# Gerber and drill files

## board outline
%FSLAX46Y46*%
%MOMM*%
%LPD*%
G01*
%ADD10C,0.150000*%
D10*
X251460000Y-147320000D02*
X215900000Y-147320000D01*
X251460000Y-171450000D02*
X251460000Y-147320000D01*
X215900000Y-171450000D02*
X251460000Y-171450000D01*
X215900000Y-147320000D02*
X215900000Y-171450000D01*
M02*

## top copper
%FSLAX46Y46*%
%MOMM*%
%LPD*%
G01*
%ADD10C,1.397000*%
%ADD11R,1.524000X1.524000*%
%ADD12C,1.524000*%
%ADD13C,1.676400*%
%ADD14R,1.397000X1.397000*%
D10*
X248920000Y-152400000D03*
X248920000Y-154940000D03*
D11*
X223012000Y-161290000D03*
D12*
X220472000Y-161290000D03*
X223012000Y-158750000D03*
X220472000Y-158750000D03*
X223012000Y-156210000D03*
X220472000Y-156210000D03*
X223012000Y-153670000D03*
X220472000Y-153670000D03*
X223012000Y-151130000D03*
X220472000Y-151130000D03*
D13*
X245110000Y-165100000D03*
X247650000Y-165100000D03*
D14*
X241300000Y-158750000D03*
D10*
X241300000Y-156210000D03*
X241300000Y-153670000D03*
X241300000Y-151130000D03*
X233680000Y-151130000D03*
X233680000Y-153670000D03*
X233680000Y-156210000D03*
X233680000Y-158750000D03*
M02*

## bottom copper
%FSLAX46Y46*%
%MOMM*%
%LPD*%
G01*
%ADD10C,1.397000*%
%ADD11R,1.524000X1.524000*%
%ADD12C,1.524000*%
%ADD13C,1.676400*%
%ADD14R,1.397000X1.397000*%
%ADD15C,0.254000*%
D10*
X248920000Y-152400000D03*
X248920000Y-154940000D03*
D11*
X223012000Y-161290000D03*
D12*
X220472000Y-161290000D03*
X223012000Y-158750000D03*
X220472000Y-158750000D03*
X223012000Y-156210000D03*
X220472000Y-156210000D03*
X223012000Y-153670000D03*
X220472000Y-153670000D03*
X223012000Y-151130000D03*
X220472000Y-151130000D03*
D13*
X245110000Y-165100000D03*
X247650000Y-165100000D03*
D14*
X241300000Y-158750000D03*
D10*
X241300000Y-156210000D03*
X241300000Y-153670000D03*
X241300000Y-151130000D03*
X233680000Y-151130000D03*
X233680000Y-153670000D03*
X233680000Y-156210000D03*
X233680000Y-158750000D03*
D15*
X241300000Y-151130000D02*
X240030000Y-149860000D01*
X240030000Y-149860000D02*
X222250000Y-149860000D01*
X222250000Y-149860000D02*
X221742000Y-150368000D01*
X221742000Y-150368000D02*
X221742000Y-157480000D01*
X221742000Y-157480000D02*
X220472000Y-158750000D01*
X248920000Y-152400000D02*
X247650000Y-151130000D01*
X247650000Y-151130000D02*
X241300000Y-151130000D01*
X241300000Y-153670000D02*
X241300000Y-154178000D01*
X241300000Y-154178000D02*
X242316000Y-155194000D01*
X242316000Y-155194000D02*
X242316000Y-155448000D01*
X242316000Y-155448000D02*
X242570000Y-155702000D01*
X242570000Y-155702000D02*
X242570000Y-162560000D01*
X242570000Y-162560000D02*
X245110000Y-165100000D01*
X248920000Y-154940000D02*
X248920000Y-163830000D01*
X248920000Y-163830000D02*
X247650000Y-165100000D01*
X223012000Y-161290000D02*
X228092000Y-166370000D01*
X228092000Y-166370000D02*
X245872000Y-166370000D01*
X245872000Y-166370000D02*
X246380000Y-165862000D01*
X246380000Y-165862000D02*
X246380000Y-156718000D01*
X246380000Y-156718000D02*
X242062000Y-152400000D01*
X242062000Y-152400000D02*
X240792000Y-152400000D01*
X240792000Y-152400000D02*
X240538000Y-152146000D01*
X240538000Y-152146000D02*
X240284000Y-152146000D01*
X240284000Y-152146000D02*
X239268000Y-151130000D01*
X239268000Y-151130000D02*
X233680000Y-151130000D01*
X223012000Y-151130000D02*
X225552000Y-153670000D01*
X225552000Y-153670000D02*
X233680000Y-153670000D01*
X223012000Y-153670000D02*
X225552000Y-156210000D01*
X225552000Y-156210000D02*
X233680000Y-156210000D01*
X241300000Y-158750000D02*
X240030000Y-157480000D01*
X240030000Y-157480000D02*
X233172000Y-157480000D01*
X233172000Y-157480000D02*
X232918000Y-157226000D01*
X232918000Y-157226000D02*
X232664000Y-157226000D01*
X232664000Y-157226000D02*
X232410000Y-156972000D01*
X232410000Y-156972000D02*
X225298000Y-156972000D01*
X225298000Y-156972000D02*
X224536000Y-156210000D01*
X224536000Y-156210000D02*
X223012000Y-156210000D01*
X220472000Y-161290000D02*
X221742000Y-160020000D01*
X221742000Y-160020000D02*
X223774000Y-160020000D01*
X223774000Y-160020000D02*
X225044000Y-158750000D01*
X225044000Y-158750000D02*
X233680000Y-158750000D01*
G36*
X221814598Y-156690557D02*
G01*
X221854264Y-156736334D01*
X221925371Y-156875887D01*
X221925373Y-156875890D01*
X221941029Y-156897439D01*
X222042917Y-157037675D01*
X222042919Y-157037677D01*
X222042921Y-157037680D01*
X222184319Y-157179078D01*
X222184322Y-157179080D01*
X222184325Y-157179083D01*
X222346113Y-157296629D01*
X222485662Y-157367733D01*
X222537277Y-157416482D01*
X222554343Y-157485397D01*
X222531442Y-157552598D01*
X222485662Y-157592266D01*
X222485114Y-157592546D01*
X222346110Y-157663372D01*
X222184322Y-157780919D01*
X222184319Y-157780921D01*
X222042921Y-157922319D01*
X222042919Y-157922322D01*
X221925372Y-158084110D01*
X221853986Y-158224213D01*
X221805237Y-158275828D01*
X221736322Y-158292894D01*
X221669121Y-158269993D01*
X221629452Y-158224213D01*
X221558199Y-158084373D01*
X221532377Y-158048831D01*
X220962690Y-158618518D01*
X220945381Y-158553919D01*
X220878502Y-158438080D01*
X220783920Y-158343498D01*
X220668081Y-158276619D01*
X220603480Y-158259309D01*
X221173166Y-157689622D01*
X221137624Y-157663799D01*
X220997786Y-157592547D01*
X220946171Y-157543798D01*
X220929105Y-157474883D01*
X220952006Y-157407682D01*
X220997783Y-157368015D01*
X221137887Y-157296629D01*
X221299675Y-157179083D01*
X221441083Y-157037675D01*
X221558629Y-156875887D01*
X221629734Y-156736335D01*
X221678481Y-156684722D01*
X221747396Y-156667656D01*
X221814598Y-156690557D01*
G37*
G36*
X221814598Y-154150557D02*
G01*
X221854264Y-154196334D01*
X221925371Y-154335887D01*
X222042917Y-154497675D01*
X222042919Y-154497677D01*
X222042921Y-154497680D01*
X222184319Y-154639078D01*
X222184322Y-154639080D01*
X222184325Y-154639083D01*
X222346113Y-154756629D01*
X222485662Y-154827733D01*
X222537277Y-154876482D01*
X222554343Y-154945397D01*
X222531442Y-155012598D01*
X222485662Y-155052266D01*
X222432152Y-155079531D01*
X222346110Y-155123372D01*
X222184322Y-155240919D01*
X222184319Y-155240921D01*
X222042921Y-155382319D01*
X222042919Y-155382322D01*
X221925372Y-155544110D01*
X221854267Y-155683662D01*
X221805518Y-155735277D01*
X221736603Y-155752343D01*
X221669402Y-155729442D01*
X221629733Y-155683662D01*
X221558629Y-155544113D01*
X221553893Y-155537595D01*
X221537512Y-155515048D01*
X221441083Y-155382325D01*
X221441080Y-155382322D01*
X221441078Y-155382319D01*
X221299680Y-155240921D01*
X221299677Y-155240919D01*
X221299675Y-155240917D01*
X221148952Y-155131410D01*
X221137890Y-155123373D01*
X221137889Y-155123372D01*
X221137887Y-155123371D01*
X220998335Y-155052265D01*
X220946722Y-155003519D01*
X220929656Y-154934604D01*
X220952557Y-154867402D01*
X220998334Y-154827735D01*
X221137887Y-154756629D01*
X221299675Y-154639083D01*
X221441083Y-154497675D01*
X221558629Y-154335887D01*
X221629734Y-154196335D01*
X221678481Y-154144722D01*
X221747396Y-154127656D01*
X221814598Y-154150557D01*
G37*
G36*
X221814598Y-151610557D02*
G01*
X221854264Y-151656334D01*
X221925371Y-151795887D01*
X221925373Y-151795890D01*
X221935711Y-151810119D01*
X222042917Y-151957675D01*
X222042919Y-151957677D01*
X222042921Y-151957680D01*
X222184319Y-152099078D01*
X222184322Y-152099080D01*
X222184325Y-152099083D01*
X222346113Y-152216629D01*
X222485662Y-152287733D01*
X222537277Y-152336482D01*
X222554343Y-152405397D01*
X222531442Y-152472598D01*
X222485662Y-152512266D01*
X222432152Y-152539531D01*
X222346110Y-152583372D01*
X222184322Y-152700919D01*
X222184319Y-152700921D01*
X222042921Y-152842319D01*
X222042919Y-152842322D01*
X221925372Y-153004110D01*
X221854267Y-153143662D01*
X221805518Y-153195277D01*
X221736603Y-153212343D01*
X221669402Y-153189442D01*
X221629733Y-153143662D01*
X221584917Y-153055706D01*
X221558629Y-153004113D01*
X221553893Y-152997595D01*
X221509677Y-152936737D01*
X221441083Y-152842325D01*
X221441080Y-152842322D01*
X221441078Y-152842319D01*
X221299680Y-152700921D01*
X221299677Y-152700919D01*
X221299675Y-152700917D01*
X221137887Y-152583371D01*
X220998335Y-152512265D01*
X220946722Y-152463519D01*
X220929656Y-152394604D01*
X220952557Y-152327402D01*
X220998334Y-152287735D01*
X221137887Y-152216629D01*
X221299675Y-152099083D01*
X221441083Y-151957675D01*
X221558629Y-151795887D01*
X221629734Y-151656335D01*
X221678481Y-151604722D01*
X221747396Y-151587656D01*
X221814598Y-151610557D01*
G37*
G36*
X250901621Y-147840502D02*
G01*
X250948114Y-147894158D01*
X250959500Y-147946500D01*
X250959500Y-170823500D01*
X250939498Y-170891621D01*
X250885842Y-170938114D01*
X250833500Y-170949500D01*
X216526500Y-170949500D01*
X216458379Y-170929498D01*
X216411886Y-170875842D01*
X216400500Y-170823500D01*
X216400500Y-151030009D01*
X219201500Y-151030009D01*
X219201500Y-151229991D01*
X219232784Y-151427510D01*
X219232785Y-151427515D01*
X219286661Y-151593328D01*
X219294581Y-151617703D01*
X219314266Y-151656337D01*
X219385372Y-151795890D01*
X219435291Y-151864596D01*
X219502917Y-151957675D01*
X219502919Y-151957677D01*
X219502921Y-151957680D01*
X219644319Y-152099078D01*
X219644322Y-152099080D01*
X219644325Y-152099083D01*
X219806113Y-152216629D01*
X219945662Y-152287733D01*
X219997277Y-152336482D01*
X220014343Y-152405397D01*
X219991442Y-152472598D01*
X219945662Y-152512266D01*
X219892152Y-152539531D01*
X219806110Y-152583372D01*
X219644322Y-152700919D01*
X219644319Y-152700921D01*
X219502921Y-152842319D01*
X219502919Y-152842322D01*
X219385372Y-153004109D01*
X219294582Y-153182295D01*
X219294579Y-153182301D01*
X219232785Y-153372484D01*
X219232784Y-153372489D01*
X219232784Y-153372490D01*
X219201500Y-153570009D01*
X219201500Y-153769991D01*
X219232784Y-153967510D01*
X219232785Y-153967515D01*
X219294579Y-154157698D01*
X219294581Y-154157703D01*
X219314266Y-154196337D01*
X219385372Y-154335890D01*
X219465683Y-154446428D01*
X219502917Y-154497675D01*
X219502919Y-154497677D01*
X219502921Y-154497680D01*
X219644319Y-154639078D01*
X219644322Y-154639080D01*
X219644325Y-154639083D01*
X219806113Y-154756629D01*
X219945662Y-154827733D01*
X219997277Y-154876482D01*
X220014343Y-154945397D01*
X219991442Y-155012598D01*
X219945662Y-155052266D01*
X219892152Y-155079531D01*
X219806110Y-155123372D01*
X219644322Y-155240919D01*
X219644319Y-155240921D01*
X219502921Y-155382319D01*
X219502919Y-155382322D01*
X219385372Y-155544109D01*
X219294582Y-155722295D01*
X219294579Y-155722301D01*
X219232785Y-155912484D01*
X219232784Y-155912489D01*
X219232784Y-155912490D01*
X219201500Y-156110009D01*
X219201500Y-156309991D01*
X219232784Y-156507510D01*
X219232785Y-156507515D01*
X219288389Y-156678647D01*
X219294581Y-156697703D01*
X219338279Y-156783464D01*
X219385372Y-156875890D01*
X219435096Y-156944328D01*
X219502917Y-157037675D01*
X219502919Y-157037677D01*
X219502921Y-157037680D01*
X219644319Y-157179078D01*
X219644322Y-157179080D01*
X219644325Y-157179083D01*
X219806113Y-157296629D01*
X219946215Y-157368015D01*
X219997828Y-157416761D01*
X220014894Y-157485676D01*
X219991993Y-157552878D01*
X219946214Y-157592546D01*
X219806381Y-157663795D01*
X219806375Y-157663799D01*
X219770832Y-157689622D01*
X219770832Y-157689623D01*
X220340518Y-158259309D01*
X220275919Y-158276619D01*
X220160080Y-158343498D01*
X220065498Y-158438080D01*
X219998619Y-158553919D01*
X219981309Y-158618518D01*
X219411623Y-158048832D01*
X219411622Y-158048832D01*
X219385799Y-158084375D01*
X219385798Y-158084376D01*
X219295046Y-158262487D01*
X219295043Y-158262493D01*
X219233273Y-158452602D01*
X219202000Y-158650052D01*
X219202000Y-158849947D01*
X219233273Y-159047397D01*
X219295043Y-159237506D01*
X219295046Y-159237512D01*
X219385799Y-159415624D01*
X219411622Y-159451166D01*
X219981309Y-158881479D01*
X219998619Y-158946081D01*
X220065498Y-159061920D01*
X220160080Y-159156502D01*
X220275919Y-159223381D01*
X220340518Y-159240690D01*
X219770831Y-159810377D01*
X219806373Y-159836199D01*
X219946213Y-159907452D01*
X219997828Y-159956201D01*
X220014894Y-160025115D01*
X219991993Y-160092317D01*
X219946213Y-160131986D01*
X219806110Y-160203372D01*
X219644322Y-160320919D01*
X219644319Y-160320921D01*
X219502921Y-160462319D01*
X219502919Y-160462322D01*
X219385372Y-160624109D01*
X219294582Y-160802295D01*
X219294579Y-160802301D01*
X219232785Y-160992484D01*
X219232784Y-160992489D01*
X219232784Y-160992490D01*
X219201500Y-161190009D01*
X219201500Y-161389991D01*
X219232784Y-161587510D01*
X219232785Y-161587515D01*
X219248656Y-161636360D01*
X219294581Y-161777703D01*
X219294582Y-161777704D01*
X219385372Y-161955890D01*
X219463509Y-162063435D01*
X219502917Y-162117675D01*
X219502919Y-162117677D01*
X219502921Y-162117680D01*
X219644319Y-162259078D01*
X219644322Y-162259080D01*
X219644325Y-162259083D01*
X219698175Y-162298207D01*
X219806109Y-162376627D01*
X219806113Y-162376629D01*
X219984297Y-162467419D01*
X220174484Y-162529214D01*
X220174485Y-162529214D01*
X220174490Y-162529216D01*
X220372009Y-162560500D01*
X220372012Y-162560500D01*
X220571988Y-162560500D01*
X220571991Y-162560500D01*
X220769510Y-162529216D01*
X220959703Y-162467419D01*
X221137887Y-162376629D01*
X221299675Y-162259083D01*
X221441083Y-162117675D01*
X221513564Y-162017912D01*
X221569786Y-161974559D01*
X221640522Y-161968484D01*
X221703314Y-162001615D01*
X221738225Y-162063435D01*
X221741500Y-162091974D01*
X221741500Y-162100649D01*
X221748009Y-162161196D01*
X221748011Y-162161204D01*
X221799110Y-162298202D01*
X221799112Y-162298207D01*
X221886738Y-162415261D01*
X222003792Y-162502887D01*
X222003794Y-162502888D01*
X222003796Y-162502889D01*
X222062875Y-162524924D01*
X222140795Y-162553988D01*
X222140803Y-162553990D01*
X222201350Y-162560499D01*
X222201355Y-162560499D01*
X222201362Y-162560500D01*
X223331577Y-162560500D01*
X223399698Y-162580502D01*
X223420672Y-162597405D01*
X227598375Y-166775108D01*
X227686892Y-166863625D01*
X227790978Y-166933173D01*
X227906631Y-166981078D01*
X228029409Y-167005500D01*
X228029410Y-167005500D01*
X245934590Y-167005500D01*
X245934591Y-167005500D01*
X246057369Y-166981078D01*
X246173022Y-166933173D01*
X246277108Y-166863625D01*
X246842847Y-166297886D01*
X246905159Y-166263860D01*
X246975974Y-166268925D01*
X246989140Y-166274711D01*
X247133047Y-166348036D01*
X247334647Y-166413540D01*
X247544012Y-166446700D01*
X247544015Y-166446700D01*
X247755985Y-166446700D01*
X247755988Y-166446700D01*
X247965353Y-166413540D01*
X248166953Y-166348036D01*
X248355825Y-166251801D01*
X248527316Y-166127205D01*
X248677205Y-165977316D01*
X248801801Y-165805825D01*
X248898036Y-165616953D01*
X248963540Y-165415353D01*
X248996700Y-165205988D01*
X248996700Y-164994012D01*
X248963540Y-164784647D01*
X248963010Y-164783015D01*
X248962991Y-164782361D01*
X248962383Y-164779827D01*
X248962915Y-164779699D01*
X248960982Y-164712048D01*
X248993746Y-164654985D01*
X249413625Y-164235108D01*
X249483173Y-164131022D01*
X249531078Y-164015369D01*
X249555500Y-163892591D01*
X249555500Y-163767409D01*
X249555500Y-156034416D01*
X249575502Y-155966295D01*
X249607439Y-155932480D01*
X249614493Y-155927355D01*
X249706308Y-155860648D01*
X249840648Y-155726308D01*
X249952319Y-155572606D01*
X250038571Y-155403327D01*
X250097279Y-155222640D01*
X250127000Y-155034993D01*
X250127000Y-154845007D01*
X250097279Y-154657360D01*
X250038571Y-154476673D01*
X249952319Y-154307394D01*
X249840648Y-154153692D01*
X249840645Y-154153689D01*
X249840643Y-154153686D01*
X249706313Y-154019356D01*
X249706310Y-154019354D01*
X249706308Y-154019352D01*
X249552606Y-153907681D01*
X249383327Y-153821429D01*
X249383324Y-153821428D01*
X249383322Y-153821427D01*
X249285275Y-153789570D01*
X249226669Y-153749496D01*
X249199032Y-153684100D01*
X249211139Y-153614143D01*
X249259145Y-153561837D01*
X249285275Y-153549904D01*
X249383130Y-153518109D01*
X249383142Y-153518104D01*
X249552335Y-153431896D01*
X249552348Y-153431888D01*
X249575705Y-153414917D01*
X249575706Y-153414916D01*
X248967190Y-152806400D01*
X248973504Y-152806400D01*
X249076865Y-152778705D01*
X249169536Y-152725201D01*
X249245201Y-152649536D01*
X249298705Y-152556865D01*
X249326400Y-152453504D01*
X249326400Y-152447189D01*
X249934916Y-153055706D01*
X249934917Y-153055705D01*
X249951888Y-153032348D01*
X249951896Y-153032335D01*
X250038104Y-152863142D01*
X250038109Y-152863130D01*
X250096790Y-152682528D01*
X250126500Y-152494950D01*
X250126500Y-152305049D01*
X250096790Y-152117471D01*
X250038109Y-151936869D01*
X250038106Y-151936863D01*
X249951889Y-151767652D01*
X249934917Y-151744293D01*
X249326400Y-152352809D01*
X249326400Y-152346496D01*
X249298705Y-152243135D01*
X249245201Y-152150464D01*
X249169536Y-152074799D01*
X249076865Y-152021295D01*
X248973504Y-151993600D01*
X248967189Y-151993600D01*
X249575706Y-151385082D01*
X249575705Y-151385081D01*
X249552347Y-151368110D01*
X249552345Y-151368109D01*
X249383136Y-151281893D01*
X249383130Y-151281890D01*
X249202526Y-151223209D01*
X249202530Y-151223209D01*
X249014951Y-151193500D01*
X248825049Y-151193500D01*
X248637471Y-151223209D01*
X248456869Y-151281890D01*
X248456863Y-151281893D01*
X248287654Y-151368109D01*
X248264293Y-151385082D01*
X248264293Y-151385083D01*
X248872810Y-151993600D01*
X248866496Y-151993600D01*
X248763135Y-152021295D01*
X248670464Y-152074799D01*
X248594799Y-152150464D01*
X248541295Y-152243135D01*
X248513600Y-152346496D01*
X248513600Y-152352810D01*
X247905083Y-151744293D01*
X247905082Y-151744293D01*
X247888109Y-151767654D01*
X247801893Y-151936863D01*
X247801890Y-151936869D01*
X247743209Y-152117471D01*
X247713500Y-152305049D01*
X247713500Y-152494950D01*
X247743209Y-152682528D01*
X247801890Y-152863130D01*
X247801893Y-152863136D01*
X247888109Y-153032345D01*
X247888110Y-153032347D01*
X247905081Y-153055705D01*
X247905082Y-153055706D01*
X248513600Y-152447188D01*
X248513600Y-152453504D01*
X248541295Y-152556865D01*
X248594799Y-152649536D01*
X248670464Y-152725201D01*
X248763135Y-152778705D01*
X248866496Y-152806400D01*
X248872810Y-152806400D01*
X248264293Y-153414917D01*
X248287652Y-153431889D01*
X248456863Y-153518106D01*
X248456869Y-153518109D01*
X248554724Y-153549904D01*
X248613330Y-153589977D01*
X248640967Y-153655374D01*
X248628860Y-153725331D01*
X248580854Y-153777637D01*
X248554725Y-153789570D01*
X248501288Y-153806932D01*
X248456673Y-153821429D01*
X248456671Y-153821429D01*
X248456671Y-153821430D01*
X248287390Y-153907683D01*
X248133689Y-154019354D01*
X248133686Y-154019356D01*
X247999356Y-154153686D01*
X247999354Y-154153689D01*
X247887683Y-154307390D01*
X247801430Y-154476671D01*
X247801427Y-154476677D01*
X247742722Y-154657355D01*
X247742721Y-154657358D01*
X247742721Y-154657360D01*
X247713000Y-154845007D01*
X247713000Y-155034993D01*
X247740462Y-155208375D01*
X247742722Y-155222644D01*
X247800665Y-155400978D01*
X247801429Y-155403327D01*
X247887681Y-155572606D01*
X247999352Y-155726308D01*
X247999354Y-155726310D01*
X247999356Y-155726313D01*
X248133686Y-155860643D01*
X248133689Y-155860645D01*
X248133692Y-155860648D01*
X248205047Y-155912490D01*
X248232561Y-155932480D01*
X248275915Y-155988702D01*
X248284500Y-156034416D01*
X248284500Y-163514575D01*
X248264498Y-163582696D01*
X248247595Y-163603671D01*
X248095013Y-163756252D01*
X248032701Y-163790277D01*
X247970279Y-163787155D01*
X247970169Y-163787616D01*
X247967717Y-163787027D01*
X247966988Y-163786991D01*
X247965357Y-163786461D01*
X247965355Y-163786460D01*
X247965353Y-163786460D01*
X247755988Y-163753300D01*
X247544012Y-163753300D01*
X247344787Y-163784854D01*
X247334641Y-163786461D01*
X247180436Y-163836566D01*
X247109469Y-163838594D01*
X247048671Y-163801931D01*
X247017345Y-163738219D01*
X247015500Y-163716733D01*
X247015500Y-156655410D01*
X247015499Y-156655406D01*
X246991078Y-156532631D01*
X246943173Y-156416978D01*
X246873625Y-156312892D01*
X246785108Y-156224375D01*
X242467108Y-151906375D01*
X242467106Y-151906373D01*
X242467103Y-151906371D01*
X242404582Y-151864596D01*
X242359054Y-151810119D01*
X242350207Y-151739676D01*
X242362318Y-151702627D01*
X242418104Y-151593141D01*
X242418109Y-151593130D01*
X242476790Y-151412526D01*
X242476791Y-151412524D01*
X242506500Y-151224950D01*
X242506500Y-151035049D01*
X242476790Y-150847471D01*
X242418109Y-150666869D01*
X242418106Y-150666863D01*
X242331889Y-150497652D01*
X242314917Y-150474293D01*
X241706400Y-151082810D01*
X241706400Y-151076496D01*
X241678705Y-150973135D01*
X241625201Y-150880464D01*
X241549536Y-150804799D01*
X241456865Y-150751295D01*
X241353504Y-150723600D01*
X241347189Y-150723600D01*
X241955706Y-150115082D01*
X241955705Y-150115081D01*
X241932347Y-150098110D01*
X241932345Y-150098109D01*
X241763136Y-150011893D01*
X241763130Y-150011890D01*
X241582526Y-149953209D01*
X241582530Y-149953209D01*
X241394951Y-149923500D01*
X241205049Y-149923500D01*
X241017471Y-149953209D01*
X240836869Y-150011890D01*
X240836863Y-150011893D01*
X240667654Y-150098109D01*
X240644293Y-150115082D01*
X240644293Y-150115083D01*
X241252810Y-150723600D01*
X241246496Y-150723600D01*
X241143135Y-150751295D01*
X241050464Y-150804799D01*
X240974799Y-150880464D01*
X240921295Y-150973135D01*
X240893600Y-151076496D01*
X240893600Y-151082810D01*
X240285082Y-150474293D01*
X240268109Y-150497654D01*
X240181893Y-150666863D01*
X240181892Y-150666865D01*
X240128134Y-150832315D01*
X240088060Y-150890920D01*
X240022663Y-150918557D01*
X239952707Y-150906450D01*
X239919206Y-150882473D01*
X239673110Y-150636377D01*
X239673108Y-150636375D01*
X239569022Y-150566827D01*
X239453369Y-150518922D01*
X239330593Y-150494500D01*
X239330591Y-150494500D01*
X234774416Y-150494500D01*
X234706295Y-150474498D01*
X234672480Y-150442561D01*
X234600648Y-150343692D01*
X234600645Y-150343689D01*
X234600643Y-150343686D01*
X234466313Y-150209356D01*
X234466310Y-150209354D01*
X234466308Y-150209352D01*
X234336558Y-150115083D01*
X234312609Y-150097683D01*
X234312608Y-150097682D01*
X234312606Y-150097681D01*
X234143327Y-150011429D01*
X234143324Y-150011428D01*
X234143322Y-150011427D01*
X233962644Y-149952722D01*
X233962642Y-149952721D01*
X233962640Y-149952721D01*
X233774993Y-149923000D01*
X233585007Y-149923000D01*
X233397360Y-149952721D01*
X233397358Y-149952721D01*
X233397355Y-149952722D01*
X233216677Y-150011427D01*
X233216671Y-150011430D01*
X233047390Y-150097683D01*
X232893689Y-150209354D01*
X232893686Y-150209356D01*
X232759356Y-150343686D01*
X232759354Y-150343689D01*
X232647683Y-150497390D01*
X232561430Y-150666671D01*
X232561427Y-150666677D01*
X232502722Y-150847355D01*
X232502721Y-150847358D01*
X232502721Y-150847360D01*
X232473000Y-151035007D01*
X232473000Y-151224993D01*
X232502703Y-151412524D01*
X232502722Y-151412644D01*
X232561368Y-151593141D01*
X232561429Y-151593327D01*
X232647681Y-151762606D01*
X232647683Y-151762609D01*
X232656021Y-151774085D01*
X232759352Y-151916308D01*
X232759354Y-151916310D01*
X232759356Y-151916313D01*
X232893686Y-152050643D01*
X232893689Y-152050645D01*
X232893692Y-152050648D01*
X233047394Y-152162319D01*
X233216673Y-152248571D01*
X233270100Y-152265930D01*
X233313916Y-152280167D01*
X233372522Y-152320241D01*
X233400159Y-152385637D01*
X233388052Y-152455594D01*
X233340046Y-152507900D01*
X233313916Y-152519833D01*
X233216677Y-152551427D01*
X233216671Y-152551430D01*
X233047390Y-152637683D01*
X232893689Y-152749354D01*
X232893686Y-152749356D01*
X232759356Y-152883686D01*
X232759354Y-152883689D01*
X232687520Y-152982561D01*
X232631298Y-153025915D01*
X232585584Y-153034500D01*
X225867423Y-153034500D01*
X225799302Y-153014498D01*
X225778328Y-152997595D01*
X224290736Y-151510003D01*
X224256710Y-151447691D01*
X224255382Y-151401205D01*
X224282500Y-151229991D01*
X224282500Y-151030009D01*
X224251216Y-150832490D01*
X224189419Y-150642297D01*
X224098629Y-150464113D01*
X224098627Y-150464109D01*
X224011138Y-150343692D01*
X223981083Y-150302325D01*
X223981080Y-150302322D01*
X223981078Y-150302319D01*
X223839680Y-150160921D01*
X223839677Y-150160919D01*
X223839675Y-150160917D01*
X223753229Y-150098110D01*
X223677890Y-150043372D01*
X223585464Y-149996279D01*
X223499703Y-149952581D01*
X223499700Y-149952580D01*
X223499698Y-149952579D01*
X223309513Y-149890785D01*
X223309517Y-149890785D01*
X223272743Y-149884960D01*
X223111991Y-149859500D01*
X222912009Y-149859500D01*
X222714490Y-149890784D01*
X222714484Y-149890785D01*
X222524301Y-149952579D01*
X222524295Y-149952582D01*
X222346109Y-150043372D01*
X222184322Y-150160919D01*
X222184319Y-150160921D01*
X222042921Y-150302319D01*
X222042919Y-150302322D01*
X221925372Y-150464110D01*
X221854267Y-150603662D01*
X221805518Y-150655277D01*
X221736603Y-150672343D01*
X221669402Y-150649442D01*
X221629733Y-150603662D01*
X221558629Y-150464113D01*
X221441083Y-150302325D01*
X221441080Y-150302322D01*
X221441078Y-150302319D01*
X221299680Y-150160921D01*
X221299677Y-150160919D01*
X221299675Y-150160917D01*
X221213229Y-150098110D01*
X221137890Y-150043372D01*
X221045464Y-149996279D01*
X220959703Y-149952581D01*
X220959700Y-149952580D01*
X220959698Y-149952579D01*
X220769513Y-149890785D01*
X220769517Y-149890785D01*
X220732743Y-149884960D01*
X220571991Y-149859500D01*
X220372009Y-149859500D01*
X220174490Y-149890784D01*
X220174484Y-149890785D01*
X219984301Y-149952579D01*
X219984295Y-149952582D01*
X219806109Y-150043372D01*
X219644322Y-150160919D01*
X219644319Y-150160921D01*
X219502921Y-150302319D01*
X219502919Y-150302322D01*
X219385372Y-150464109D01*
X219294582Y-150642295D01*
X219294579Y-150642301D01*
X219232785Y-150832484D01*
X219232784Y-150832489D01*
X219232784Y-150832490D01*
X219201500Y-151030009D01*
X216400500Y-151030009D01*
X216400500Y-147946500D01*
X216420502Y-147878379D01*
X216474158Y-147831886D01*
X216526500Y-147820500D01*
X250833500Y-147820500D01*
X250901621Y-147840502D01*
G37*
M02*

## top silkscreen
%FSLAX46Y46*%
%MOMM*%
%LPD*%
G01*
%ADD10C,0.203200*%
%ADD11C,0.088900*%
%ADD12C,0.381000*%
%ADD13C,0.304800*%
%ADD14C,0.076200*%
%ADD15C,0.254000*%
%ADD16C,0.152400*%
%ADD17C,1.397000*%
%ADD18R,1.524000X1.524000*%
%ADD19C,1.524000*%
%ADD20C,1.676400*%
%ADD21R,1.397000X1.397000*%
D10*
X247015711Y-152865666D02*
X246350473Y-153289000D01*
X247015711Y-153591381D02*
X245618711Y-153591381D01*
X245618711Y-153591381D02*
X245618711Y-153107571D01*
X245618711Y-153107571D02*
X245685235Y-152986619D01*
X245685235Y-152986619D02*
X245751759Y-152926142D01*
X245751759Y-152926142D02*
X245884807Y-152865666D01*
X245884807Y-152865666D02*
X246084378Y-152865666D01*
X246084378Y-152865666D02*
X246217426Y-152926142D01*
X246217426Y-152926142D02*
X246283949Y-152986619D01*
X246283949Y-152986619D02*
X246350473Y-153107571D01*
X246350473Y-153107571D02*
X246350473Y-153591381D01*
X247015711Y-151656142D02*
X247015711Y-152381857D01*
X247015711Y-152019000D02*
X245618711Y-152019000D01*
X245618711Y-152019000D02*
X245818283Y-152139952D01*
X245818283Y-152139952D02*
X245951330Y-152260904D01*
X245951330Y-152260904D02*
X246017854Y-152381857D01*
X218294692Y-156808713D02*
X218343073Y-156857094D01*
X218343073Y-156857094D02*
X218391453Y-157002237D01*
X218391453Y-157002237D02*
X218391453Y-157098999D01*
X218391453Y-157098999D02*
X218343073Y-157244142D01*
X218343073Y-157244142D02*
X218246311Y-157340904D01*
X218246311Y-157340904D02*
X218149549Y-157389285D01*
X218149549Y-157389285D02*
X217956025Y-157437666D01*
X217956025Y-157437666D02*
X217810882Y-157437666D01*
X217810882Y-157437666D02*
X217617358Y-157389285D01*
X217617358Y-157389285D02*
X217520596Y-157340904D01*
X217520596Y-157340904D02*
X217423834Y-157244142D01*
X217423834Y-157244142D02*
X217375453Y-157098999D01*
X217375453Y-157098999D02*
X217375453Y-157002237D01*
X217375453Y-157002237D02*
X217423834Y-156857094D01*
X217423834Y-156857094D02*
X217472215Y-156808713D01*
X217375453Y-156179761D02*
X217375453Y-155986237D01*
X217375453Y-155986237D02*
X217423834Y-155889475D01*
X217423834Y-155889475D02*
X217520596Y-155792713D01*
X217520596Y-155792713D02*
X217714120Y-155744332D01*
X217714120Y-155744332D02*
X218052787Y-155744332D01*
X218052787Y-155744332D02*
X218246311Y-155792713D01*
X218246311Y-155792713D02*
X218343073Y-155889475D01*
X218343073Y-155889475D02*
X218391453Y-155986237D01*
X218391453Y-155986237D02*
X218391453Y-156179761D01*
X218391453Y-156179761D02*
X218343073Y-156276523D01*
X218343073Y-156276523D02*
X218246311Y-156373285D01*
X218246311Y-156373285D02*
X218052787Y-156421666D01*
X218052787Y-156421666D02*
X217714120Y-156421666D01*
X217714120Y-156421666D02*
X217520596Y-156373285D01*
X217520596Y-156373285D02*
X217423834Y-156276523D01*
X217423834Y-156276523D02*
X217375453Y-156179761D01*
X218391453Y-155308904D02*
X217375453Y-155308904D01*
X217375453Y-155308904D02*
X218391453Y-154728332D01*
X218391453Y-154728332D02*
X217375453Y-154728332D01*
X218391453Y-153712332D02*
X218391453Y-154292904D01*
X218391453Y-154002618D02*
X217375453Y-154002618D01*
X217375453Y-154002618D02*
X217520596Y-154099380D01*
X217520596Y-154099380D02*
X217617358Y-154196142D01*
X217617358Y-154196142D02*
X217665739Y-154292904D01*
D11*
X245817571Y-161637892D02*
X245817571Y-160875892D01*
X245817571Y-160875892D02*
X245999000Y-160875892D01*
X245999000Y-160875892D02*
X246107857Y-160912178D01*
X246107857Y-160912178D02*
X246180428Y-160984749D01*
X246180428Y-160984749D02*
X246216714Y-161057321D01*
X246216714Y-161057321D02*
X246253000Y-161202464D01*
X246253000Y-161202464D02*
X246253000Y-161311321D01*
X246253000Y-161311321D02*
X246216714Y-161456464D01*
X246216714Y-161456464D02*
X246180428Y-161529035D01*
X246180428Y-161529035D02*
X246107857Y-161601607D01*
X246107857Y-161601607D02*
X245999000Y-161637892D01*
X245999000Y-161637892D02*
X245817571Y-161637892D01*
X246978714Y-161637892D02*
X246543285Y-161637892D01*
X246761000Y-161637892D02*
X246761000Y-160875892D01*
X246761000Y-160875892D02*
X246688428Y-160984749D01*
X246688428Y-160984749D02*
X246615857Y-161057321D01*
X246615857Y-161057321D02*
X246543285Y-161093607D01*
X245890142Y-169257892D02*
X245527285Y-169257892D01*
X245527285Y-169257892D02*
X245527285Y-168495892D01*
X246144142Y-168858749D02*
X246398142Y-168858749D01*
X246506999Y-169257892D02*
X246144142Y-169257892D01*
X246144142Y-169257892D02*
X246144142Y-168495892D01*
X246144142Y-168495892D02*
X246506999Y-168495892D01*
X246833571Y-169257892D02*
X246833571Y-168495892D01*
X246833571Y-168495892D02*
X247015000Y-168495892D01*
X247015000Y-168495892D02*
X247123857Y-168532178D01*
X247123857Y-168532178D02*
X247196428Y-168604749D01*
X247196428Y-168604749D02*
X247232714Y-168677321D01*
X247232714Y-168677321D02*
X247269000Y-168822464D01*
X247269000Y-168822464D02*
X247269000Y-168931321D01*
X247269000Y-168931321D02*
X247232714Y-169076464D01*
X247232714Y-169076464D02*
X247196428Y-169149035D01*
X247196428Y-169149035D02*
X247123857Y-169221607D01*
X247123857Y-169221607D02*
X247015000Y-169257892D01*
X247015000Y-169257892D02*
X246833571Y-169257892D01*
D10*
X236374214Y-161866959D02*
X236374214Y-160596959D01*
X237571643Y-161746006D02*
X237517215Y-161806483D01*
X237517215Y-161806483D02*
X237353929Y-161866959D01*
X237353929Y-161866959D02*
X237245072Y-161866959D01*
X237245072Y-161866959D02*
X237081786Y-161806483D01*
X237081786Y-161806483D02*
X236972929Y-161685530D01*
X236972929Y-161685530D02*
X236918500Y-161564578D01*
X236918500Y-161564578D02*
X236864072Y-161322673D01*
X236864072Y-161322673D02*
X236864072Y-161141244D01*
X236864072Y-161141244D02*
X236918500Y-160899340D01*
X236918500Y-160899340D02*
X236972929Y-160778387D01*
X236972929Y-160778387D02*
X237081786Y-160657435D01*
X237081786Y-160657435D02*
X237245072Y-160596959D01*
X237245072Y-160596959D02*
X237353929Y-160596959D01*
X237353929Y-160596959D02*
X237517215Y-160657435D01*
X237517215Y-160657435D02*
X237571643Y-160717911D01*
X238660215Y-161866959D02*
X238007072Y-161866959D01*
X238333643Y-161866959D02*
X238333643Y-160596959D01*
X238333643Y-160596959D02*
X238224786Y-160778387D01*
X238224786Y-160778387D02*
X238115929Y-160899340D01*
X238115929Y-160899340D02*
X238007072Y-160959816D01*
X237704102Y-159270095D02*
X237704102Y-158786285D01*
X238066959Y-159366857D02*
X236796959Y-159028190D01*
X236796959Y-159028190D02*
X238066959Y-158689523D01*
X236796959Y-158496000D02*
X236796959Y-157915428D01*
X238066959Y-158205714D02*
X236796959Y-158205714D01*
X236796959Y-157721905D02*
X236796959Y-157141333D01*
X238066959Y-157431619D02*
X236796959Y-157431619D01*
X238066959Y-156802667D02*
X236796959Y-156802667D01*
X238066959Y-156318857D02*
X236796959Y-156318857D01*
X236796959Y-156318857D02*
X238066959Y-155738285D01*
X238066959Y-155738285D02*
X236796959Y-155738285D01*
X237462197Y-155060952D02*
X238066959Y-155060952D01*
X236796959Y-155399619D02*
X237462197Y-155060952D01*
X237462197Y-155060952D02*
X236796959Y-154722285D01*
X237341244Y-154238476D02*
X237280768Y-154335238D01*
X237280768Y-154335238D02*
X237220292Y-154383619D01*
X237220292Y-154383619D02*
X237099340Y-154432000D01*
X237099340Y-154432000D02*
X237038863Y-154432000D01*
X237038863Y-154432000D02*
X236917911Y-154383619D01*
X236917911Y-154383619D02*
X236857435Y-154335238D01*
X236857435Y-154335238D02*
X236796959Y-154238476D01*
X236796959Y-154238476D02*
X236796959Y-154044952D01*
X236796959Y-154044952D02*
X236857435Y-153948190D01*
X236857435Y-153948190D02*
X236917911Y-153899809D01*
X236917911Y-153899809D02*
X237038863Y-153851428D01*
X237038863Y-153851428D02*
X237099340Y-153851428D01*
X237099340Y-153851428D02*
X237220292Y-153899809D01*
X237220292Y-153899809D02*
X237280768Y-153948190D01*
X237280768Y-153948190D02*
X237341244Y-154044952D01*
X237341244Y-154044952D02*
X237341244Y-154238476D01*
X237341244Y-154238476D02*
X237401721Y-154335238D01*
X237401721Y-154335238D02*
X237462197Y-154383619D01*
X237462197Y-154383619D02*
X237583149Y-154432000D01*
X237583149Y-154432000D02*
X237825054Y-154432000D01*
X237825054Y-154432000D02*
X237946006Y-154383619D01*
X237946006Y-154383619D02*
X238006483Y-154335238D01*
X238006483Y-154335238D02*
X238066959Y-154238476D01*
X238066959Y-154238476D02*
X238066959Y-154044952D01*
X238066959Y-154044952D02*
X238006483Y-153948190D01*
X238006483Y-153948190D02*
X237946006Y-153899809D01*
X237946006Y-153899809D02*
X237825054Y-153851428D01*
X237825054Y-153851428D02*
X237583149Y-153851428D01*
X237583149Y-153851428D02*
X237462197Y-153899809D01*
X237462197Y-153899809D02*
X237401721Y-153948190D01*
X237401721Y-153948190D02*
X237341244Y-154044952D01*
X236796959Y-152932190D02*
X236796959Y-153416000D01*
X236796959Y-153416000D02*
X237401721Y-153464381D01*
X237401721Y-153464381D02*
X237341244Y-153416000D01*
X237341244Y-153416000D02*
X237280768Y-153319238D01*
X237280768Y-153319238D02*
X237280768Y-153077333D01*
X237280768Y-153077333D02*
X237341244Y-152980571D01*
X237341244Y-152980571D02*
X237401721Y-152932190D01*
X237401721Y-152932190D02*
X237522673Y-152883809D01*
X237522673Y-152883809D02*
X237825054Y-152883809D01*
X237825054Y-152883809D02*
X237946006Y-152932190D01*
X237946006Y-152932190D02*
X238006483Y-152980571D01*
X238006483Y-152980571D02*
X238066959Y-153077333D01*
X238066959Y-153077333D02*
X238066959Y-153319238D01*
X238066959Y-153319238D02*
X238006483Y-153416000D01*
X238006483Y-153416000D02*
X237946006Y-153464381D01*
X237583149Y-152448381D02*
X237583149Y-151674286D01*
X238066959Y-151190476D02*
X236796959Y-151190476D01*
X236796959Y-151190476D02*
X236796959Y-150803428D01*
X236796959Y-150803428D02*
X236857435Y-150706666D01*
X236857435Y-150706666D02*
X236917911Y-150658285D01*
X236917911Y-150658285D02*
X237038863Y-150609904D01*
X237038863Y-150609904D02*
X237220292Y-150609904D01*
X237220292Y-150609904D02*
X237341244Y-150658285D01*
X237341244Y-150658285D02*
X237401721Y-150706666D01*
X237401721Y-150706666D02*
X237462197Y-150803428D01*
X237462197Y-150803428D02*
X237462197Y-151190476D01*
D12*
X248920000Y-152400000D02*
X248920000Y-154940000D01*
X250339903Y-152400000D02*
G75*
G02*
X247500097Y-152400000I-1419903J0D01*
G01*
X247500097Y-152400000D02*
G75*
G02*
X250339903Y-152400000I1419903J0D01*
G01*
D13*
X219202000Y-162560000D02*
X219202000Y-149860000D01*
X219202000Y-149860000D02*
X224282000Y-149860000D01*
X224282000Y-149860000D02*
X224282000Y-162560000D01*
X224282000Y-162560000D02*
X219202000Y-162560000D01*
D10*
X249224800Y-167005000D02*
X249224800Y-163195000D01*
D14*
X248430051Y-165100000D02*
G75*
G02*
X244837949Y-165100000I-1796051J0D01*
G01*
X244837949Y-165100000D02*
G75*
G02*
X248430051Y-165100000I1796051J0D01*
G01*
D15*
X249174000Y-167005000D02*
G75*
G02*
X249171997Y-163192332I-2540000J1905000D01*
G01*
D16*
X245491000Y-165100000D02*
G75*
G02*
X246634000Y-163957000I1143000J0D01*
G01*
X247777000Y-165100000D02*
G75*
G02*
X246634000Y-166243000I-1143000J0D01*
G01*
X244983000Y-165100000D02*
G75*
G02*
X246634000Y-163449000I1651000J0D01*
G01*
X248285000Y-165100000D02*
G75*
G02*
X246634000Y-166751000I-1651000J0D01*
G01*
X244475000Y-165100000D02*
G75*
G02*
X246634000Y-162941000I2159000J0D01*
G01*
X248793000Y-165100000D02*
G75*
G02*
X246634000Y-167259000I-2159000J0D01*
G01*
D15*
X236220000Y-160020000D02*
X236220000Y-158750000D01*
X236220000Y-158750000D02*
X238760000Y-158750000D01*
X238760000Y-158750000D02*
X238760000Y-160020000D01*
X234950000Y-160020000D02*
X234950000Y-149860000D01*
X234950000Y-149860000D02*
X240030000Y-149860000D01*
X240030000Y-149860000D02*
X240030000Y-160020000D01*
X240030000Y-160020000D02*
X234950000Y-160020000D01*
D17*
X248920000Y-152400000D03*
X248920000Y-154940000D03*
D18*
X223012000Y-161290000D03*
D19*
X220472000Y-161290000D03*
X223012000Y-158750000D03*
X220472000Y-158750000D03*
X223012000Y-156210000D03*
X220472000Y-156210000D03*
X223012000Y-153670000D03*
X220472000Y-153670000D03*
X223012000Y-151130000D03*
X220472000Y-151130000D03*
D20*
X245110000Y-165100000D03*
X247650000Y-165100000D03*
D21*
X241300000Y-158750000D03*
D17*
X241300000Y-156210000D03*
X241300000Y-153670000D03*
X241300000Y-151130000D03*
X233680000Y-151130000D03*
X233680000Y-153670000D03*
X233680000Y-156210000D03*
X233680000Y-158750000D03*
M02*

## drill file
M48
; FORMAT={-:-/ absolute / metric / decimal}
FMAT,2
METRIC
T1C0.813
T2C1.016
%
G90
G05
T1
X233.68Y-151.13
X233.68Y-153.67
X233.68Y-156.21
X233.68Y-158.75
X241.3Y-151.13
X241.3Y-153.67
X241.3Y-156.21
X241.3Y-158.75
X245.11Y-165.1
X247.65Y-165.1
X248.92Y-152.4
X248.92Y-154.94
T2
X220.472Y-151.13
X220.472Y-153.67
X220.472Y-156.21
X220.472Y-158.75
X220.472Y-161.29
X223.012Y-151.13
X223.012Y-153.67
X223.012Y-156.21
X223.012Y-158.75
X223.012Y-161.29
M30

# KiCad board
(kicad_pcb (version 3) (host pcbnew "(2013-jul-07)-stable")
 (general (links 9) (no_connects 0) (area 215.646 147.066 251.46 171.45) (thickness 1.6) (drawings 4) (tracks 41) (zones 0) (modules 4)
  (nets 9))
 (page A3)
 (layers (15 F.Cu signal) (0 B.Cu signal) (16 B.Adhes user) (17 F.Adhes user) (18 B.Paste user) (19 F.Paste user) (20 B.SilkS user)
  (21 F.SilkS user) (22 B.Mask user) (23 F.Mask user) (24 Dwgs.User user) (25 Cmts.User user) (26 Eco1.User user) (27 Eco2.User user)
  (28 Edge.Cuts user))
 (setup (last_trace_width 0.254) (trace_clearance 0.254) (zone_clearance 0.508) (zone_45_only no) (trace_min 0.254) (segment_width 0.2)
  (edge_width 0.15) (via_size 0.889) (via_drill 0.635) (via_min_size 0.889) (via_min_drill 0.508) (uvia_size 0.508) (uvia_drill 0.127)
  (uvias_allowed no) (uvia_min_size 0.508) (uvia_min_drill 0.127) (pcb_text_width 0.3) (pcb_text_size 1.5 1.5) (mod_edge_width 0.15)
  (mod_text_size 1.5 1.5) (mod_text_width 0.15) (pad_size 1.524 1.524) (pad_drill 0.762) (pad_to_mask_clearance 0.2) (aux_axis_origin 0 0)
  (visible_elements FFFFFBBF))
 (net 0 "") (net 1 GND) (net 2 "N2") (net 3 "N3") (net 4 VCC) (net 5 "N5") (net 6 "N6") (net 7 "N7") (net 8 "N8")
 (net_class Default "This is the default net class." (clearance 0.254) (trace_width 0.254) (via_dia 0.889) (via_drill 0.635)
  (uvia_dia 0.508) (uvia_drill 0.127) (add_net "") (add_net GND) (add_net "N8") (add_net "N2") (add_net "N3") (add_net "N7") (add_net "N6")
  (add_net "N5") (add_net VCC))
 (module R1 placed (layer F.Cu) (at 248.92 153.67 270) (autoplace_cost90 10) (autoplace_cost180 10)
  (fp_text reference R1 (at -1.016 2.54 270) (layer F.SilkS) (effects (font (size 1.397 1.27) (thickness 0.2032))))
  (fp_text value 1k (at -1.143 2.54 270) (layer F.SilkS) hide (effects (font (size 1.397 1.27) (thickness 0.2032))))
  (fp_line (start -1.27 0) (end 1.27 0) (layer F.SilkS) (width 0.381))
  (fp_circle (center -1.27 0) (end -0.635 1.27) (layer F.SilkS) (width 0.381))
  (pad 1 thru_hole circle (at -1.27 0 270) (size 1.397 1.397) (drill 0.8128) (layers *.Cu *.Mask F.SilkS) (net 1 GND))
  (pad 2 thru_hole circle (at 1.27 0 270) (size 1.397 1.397) (drill 0.8128) (layers *.Cu *.Mask F.SilkS) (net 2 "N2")))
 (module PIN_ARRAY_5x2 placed (layer F.Cu) (at 221.742 156.21 90)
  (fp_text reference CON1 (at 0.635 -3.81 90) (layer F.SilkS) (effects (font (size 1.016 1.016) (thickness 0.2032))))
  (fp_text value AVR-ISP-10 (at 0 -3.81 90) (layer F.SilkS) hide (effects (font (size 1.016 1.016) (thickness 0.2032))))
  (fp_line (start -6.35 -2.54) (end 6.35 -2.54) (layer F.SilkS) (width 0.3048))
  (fp_line (start 6.35 -2.54) (end 6.35 2.54) (layer F.SilkS) (width 0.3048))
  (fp_line (start 6.35 2.54) (end -6.35 2.54) (layer F.SilkS) (width 0.3048))
  (fp_line (start -6.35 2.54) (end -6.35 -2.54) (layer F.SilkS) (width 0.3048))
  (pad 1 thru_hole rect (at -5.08 1.27 90) (size 1.524 1.524) (drill 1.016) (layers *.Cu *.Mask F.SilkS) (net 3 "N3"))
  (pad 2 thru_hole circle (at -5.08 -1.27 90) (size 1.524 1.524) (drill 1.016) (layers *.Cu *.Mask F.SilkS) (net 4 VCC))
  (pad 3 thru_hole circle (at -2.54 1.27 90) (size 1.524 1.524) (drill 1.016) (layers *.Cu *.Mask F.SilkS))
  (pad 4 thru_hole circle (at -2.54 -1.27 90) (size 1.524 1.524) (drill 1.016) (layers *.Cu *.Mask F.SilkS) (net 1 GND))
  (pad 5 thru_hole circle (at 0 1.27 90) (size 1.524 1.524) (drill 1.016) (layers *.Cu *.Mask F.SilkS) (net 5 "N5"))
  (pad 6 thru_hole circle (at 0 -1.27 90) (size 1.524 1.524) (drill 1.016) (layers *.Cu *.Mask F.SilkS))
  (pad 7 thru_hole circle (at 2.54 1.27 90) (size 1.524 1.524) (drill 1.016) (layers *.Cu *.Mask F.SilkS) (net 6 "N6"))
  (pad 8 thru_hole circle (at 2.54 -1.27 90) (size 1.524 1.524) (drill 1.016) (layers *.Cu *.Mask F.SilkS))
  (pad 9 thru_hole circle (at 5.08 1.27 90) (size 1.524 1.524) (drill 1.016) (layers *.Cu *.Mask F.SilkS) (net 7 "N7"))
  (pad 10 thru_hole circle (at 5.08 -1.27 90) (size 1.524 1.524) (drill 1.016) (layers *.Cu *.Mask F.SilkS)))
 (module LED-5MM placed (layer F.Cu) (at 246.38 165.1)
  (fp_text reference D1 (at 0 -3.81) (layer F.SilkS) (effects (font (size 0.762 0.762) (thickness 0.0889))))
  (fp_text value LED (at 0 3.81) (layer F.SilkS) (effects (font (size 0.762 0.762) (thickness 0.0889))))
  (fp_line (start 2.8448 1.905) (end 2.8448 -1.905) (layer F.SilkS) (width 0.2032))
  (fp_circle (center 0.254 0) (end -1.016 1.27) (layer F.SilkS) (width 0.0762))
  (fp_arc (start 0.254 0) (end 2.794 1.905) (angle 286.2) (layer F.SilkS) (width 0.254))
  (fp_arc (start 0.254 0) (end -0.889 0) (angle 90) (layer F.SilkS) (width 0.1524))
  (fp_arc (start 0.254 0) (end 1.397 0) (angle 90) (layer F.SilkS) (width 0.1524))
  (fp_arc (start 0.254 0) (end -1.397 0) (angle 90) (layer F.SilkS) (width 0.1524))
  (fp_arc (start 0.254 0) (end 1.905 0) (angle 90) (layer F.SilkS) (width 0.1524))
  (fp_arc (start 0.254 0) (end -1.905 0) (angle 90) (layer F.SilkS) (width 0.1524))
  (fp_arc (start 0.254 0) (end 2.413 0) (angle 90) (layer F.SilkS) (width 0.1524))
  (pad 1 thru_hole circle (at -1.27 0) (size 1.6764 1.6764) (drill 0.8128) (layers *.Cu *.Mask F.SilkS) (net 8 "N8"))
  (pad 2 thru_hole circle (at 1.27 0) (size 1.6764 1.6764) (drill 0.8128) (layers *.Cu *.Mask F.SilkS) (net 2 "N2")))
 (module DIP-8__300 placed (layer F.Cu) (at 237.49 154.94 90)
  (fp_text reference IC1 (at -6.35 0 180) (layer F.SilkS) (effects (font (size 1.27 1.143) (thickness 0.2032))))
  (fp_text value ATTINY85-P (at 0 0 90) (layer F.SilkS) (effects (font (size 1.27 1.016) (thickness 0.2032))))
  (fp_line (start -5.08 -1.27) (end -3.81 -1.27) (layer F.SilkS) (width 0.254))
  (fp_line (start -3.81 -1.27) (end -3.81 1.27) (layer F.SilkS) (width 0.254))
  (fp_line (start -3.81 1.27) (end -5.08 1.27) (layer F.SilkS) (width 0.254))
  (fp_line (start -5.08 -2.54) (end 5.08 -2.54) (layer F.SilkS) (width 0.254))
  (fp_line (start 5.08 -2.54) (end 5.08 2.54) (layer F.SilkS) (width 0.254))
  (fp_line (start 5.08 2.54) (end -5.08 2.54) (layer F.SilkS) (width 0.254))
  (fp_line (start -5.08 2.54) (end -5.08 -2.54) (layer F.SilkS) (width 0.254))
  (pad 1 thru_hole rect (at -3.81 3.81 90) (size 1.397 1.397) (drill 0.8128) (layers *.Cu *.Mask F.SilkS) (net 5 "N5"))
  (pad 2 thru_hole circle (at -1.27 3.81 90) (size 1.397 1.397) (drill 0.8128) (layers *.Cu *.Mask F.SilkS))
  (pad 3 thru_hole circle (at 1.27 3.81 90) (size 1.397 1.397) (drill 0.8128) (layers *.Cu *.Mask F.SilkS) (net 8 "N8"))
  (pad 4 thru_hole circle (at 3.81 3.81 90) (size 1.397 1.397) (drill 0.8128) (layers *.Cu *.Mask F.SilkS) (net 1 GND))
  (pad 5 thru_hole circle (at 3.81 -3.81 90) (size 1.397 1.397) (drill 0.8128) (layers *.Cu *.Mask F.SilkS) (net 3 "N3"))
  (pad 6 thru_hole circle (at 1.27 -3.81 90) (size 1.397 1.397) (drill 0.8128) (layers *.Cu *.Mask F.SilkS) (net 7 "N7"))
  (pad 7 thru_hole circle (at -1.27 -3.81 90) (size 1.397 1.397) (drill 0.8128) (layers *.Cu *.Mask F.SilkS) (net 6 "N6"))
  (pad 8 thru_hole circle (at -3.81 -3.81 90) (size 1.397 1.397) (drill 0.8128) (layers *.Cu *.Mask F.SilkS) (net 4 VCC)))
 (gr_line (start 251.46 147.32) (end 215.9 147.32) (angle 90) (layer Edge.Cuts) (width 0.15))
 (gr_line (start 251.46 171.45) (end 251.46 147.32) (angle 90) (layer Edge.Cuts) (width 0.15))
 (gr_line (start 215.9 171.45) (end 251.46 171.45) (angle 90) (layer Edge.Cuts) (width 0.15))
 (gr_line (start 215.9 147.32) (end 215.9 171.45) (angle 90) (layer Edge.Cuts) (width 0.15))
 (segment (start 241.3 151.13) (end 240.03 149.86) (width 0.254) (layer B.Cu) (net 1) (status 80000))
 (segment (start 240.03 149.86) (end 222.25 149.86) (width 0.254) (layer B.Cu) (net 1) (status 80000))
 (segment (start 222.25 149.86) (end 221.742 150.368) (width 0.254) (layer B.Cu) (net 1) (status 80000))
 (segment (start 221.742 150.368) (end 221.742 157.48) (width 0.254) (layer B.Cu) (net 1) (status 80000))
 (segment (start 221.742 157.48) (end 220.472 158.75) (width 0.254) (layer B.Cu) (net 1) (status 80000))
 (segment (start 248.92 152.4) (end 247.65 151.13) (width 0.254) (layer B.Cu) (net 1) (status 80000))
 (segment (start 247.65 151.13) (end 241.3 151.13) (width 0.254) (layer B.Cu) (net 1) (status 80000))
 (segment (start 241.3 153.67) (end 241.3 154.178) (width 0.254) (layer B.Cu) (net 8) (status 80000))
 (segment (start 241.3 154.178) (end 242.316 155.194) (width 0.254) (layer B.Cu) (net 8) (status 80000))
 (segment (start 242.316 155.194) (end 242.316 155.448) (width 0.254) (layer B.Cu) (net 8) (status 80000))
 (segment (start 242.316 155.448) (end 242.57 155.702) (width 0.254) (layer B.Cu) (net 8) (status 80000))
 (segment (start 242.57 155.702) (end 242.57 162.56) (width 0.254) (layer B.Cu) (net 8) (status 80000))
 (segment (start 242.57 162.56) (end 245.11 165.1) (width 0.254) (layer B.Cu) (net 8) (status 80000))
 (segment (start 248.92 154.94) (end 248.92 163.83) (width 0.254) (layer B.Cu) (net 2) (status 80000))
 (segment (start 248.92 163.83) (end 247.65 165.1) (width 0.254) (layer B.Cu) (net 2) (status 80000))
 (segment (start 223.012 161.29) (end 228.092 166.37) (width 0.254) (layer B.Cu) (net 3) (status 80000))
 (segment (start 228.092 166.37) (end 245.872 166.37) (width 0.254) (layer B.Cu) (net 3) (status 80000))
 (segment (start 245.872 166.37) (end 246.38 165.862) (width 0.254) (layer B.Cu) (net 3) (status 80000))
 (segment (start 246.38 165.862) (end 246.38 156.718) (width 0.254) (layer B.Cu) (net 3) (status 80000))
 (segment (start 246.38 156.718) (end 242.062 152.4) (width 0.254) (layer B.Cu) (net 3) (status 80000))
 (segment (start 242.062 152.4) (end 240.792 152.4) (width 0.254) (layer B.Cu) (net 3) (status 80000))
 (segment (start 240.792 152.4) (end 240.538 152.146) (width 0.254) (layer B.Cu) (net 3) (status 80000))
 (segment (start 240.538 152.146) (end 240.284 152.146) (width 0.254) (layer B.Cu) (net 3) (status 80000))
 (segment (start 240.284 152.146) (end 239.268 151.13) (width 0.254) (layer B.Cu) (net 3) (status 80000))
 (segment (start 239.268 151.13) (end 233.68 151.13) (width 0.254) (layer B.Cu) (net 3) (status 80000))
 (segment (start 223.012 151.13) (end 225.552 153.67) (width 0.254) (layer B.Cu) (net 7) (status 80000))
 (segment (start 225.552 153.67) (end 233.68 153.67) (width 0.254) (layer B.Cu) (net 7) (status 80000))
 (segment (start 223.012 153.67) (end 225.552 156.21) (width 0.254) (layer B.Cu) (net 6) (status 80000))
 (segment (start 225.552 156.21) (end 233.68 156.21) (width 0.254) (layer B.Cu) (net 6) (status 80000))
 (segment (start 241.3 158.75) (end 240.03 157.48) (width 0.254) (layer B.Cu) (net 5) (status 80000))
 (segment (start 240.03 157.48) (end 233.172 157.48) (width 0.254) (layer B.Cu) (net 5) (status 80000))
 (segment (start 233.172 157.48) (end 232.918 157.226) (width 0.254) (layer B.Cu) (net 5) (status 80000))
 (segment (start 232.918 157.226) (end 232.664 157.226) (width 0.254) (layer B.Cu) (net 5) (status 80000))
 (segment (start 232.664 157.226) (end 232.41 156.972) (width 0.254) (layer B.Cu) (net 5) (status 80000))
 (segment (start 232.41 156.972) (end 225.298 156.972) (width 0.254) (layer B.Cu) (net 5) (status 80000))
 (segment (start 225.298 156.972) (end 224.536 156.21) (width 0.254) (layer B.Cu) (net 5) (status 80000))
 (segment (start 224.536 156.21) (end 223.012 156.21) (width 0.254) (layer B.Cu) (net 5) (status 80000))
 (segment (start 220.472 161.29) (end 221.742 160.02) (width 0.254) (layer B.Cu) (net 4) (status 80000))
 (segment (start 221.742 160.02) (end 223.774 160.02) (width 0.254) (layer B.Cu) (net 4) (status 80000))
 (segment (start 223.774 160.02) (end 225.044 158.75) (width 0.254) (layer B.Cu) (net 4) (status 80000))
 (segment (start 225.044 158.75) (end 233.68 158.75) (width 0.254) (layer B.Cu) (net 4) (status 80000))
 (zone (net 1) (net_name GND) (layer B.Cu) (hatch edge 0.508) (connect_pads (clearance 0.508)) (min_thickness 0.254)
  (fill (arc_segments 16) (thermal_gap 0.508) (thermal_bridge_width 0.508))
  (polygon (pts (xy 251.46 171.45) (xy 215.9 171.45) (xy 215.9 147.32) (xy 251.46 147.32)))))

